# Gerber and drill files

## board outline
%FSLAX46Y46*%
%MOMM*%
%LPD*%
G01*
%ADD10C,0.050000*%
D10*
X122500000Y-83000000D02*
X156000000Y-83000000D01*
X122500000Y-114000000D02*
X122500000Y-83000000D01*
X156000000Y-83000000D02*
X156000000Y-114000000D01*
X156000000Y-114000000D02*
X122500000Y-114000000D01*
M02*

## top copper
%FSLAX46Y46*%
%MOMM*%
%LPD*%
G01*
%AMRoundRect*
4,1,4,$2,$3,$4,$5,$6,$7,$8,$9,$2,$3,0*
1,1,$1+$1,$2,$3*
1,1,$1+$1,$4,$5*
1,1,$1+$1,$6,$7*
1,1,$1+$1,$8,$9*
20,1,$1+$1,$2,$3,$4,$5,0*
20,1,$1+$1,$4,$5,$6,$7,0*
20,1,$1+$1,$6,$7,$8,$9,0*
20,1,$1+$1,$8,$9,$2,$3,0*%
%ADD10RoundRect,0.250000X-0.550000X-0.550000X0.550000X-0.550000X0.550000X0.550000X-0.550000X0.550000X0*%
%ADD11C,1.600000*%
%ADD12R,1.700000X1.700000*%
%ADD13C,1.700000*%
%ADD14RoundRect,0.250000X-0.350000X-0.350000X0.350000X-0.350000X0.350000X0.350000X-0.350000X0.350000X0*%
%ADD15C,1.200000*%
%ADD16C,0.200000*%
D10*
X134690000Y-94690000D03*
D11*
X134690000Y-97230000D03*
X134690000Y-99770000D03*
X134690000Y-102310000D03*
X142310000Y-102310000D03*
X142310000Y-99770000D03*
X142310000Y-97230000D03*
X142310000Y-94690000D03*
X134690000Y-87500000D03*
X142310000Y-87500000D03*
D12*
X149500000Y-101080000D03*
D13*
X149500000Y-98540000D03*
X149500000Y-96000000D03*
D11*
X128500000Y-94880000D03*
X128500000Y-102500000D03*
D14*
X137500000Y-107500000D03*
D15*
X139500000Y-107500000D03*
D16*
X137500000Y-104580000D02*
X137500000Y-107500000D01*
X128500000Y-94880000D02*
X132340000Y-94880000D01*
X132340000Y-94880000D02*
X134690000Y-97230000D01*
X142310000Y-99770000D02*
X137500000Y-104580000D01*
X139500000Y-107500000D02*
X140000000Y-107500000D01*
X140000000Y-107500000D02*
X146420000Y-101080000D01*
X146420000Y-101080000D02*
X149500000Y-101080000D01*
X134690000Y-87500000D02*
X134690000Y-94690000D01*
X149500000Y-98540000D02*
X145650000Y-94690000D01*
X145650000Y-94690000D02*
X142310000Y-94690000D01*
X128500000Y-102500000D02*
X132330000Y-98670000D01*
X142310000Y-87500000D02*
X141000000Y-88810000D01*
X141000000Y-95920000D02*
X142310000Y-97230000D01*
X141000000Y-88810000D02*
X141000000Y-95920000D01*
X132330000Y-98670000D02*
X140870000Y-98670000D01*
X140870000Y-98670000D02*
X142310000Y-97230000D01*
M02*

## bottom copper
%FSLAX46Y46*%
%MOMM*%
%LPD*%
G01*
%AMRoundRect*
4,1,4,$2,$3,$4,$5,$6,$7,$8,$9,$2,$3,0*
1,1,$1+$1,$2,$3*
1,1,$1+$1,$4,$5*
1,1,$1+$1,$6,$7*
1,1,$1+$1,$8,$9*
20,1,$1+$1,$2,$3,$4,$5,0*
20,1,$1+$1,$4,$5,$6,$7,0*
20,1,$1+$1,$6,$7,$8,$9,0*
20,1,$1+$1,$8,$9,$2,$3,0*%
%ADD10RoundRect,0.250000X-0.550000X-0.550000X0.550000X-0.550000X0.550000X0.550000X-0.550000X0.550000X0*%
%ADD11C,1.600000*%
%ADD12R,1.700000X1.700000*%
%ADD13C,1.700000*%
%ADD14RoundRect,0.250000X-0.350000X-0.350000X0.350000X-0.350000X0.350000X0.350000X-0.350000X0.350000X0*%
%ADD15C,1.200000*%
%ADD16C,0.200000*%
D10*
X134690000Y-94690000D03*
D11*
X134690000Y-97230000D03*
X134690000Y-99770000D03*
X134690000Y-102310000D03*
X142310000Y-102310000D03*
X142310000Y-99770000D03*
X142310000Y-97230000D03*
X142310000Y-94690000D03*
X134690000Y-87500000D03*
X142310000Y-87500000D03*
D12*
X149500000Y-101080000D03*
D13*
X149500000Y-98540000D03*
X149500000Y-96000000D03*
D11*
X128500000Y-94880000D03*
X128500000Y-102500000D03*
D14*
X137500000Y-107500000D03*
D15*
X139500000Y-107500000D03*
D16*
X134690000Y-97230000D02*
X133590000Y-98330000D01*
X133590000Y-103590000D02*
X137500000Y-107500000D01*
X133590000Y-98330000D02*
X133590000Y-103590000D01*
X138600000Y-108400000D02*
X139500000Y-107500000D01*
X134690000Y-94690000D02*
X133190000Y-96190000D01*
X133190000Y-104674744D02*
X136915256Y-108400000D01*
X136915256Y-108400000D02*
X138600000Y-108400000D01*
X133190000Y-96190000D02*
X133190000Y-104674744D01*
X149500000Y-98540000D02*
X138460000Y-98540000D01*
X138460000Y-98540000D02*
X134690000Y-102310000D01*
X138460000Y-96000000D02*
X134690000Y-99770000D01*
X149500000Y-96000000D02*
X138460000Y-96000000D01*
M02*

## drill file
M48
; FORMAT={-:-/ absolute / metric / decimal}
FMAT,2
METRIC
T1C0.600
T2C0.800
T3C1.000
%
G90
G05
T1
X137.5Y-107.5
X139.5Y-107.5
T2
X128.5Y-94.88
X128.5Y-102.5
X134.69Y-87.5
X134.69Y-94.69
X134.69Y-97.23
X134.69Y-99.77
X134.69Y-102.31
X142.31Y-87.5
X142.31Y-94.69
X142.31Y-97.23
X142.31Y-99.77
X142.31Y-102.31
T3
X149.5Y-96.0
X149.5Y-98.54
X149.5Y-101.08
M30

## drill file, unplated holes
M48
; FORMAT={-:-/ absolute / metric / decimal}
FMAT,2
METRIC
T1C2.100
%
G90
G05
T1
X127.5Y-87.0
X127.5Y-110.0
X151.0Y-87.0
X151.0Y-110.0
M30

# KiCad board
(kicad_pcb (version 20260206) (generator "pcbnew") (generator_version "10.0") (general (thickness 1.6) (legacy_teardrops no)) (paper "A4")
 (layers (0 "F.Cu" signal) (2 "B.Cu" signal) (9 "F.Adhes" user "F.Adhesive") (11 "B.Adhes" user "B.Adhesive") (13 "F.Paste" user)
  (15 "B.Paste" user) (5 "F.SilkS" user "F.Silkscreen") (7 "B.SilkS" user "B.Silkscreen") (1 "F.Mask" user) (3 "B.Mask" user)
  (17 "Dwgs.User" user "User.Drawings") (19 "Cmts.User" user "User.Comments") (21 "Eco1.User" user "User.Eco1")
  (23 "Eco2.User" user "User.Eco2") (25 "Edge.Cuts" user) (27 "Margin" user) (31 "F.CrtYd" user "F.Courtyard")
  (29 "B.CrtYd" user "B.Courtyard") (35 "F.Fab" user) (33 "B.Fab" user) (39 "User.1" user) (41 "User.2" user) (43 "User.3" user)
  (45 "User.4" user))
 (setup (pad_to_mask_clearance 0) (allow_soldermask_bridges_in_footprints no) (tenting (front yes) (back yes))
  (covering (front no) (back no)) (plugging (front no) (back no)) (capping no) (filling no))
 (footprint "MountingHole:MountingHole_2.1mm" (layer "F.Cu") (at 151 110)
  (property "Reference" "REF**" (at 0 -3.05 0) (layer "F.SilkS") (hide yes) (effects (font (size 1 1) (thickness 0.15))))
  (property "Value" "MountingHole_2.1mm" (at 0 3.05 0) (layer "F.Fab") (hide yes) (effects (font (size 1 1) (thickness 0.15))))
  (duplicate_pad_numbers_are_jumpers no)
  (pad "" np_thru_hole circle (at 0 0) (size 2.1 2.1) (drill 2.1) (layers "*.Cu" "*.Mask")))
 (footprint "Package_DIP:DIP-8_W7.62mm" (layer "F.Cu") (at 134.69 94.69)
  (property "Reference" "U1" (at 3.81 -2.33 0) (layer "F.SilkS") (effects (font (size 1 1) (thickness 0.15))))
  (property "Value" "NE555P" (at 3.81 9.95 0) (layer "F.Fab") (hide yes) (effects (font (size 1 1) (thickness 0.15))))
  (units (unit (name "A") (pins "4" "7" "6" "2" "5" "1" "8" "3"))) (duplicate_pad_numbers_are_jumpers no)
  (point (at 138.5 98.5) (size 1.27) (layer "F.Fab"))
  (pad "1" thru_hole roundrect (at 0 0) (size 1.6 1.6) (drill 0.8) (layers "*.Cu" "*.Mask") (remove_unused_layers no)
   (roundrect_rratio 0.15625) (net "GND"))
  (pad "2" thru_hole circle (at 0 2.54) (size 1.6 1.6) (drill 0.8) (layers "*.Cu" "*.Mask") (remove_unused_layers no) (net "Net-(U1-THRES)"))
  (pad "3" thru_hole circle (at 0 5.08) (size 1.6 1.6) (drill 0.8) (layers "*.Cu" "*.Mask") (remove_unused_layers no) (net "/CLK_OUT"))
  (pad "4" thru_hole circle (at 0 7.62) (size 1.6 1.6) (drill 0.8) (layers "*.Cu" "*.Mask") (remove_unused_layers no) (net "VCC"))
  (pad "5" thru_hole circle (at 7.62 7.62) (size 1.6 1.6) (drill 0.8) (layers "*.Cu" "*.Mask") (remove_unused_layers no)
   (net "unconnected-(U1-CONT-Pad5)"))
  (pad "6" thru_hole circle (at 7.62 5.08) (size 1.6 1.6) (drill 0.8) (layers "*.Cu" "*.Mask") (remove_unused_layers no)
   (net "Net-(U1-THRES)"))
  (pad "7" thru_hole circle (at 7.62 2.54) (size 1.6 1.6) (drill 0.8) (layers "*.Cu" "*.Mask") (remove_unused_layers no)
   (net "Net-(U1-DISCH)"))
  (pad "8" thru_hole circle (at 7.62 0) (size 1.6 1.6) (drill 0.8) (layers "*.Cu" "*.Mask") (remove_unused_layers no) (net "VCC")))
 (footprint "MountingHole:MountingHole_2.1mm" (layer "F.Cu") (at 151 87)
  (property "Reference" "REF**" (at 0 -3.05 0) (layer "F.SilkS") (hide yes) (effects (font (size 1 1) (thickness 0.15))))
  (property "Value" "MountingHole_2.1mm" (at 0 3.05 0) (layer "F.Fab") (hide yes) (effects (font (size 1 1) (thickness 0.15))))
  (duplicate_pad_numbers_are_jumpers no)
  (pad "" np_thru_hole circle (at 0 0) (size 2.1 2.1) (drill 2.1) (layers "*.Cu" "*.Mask")))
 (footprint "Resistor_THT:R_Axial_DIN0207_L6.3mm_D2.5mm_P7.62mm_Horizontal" (layer "F.Cu") (at 134.69 87.5)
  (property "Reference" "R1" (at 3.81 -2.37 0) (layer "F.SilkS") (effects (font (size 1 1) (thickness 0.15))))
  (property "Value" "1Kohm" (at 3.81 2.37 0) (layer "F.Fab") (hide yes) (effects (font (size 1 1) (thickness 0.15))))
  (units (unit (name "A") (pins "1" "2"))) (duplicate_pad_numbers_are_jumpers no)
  (pad "1" thru_hole circle (at 0 0) (size 1.6 1.6) (drill 0.8) (layers "*.Cu" "*.Mask") (remove_unused_layers no) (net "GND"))
  (pad "2" thru_hole circle (at 7.62 0) (size 1.6 1.6) (drill 0.8) (layers "*.Cu" "*.Mask") (remove_unused_layers no) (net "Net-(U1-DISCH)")))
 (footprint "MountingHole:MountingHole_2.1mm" (layer "F.Cu") (at 127.5 110)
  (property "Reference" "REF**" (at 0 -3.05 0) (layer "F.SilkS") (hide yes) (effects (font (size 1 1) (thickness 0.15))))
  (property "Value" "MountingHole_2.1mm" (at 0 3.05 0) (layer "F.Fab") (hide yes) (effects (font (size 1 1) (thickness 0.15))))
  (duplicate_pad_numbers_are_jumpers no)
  (pad "" np_thru_hole circle (at 0 0) (size 2.1 2.1) (drill 2.1) (layers "*.Cu" "*.Mask")))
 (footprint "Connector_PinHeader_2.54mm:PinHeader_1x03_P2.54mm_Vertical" (layer "F.Cu") (at 149.5 101.08 180)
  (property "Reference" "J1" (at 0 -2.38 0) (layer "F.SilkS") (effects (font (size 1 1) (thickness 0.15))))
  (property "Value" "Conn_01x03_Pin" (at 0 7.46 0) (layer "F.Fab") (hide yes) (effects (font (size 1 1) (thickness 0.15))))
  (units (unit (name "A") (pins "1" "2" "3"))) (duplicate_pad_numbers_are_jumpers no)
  (pad "1" thru_hole rect (at 0 0 180) (size 1.7 1.7) (drill 1) (layers "*.Cu" "*.Mask") (remove_unused_layers no) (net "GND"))
  (pad "2" thru_hole circle (at 0 2.54 180) (size 1.7 1.7) (drill 1) (layers "*.Cu" "*.Mask") (remove_unused_layers no) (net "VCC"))
  (pad "3" thru_hole circle (at 0 5.08 180) (size 1.7 1.7) (drill 1) (layers "*.Cu" "*.Mask") (remove_unused_layers no) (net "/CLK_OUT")))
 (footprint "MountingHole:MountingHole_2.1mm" (layer "F.Cu") (at 127.5 87)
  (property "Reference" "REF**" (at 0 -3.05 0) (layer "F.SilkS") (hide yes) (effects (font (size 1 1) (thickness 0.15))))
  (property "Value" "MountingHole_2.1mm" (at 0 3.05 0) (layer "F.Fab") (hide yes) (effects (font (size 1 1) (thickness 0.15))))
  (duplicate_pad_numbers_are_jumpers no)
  (pad "" np_thru_hole circle (at 0 0) (size 2.1 2.1) (drill 2.1) (layers "*.Cu" "*.Mask")))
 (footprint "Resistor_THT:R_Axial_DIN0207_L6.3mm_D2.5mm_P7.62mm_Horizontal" (layer "F.Cu") (at 128.5 94.88 -90)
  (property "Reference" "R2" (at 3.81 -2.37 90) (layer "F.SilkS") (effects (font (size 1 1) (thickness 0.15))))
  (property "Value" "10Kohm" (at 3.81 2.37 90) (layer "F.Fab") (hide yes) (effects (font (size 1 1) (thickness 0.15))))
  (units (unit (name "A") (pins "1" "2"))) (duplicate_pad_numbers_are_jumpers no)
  (pad "1" thru_hole circle (at 0 0 270) (size 1.6 1.6) (drill 0.8) (layers "*.Cu" "*.Mask") (remove_unused_layers no)
   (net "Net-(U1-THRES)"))
  (pad "2" thru_hole circle (at 7.62 0 270) (size 1.6 1.6) (drill 0.8) (layers "*.Cu" "*.Mask") (remove_unused_layers no)
   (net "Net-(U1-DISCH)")))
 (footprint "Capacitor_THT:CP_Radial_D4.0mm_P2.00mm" (layer "F.Cu") (at 137.5 107.5)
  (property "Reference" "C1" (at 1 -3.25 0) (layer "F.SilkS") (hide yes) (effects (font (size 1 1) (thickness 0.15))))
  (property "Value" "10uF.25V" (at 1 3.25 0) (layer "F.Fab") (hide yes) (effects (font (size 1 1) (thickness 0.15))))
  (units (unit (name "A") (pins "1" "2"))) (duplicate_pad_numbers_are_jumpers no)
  (pad "1" thru_hole roundrect (at 0 0) (size 1.2 1.2) (drill 0.6) (layers "*.Cu" "*.Mask") (remove_unused_layers no)
   (roundrect_rratio 0.208333) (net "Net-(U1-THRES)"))
  (pad "2" thru_hole circle (at 2 0) (size 1.2 1.2) (drill 0.6) (layers "*.Cu" "*.Mask") (remove_unused_layers no) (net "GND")))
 (gr_line (start 122.5 83) (end 156 83) (stroke (width 0.05) (type default)) (layer "Edge.Cuts"))
 (gr_line (start 122.5 114) (end 122.5 83) (stroke (width 0.05) (type default)) (layer "Edge.Cuts"))
 (gr_line (start 156 83) (end 156 114) (stroke (width 0.05) (type default)) (layer "Edge.Cuts"))
 (gr_line (start 156 114) (end 122.5 114) (stroke (width 0.05) (type default)) (layer "Edge.Cuts"))
 (segment (start 139.5 107.5) (end 140 107.5) (width 0.2) (layer "F.Cu") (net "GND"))
 (segment (start 140 107.5) (end 146.42 101.08) (width 0.2) (layer "F.Cu") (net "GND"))
 (segment (start 146.42 101.08) (end 149.5 101.08) (width 0.2) (layer "F.Cu") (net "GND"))
 (segment (start 134.69 87.5) (end 134.69 94.69) (width 0.2) (layer "F.Cu") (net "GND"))
 (segment (start 138.6 108.4) (end 139.5 107.5) (width 0.2) (layer "B.Cu") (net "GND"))
 (segment (start 134.69 94.69) (end 133.19 96.19) (width 0.2) (layer "B.Cu") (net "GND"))
 (segment (start 133.19 104.674744) (end 136.915256 108.4) (width 0.2) (layer "B.Cu") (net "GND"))
 (segment (start 136.915256 108.4) (end 138.6 108.4) (width 0.2) (layer "B.Cu") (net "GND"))
 (segment (start 133.19 96.19) (end 133.19 104.674744) (width 0.2) (layer "B.Cu") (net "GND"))
 (segment (start 137.5 104.58) (end 137.5 107.5) (width 0.2) (layer "F.Cu") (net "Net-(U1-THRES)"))
 (segment (start 128.5 94.88) (end 132.34 94.88) (width 0.2) (layer "F.Cu") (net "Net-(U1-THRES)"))
 (segment (start 132.34 94.88) (end 134.69 97.23) (width 0.2) (layer "F.Cu") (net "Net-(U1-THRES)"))
 (segment (start 142.31 99.77) (end 137.5 104.58) (width 0.2) (layer "F.Cu") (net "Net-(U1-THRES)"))
 (segment (start 134.69 97.23) (end 133.59 98.33) (width 0.2) (layer "B.Cu") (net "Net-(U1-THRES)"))
 (segment (start 133.59 103.59) (end 137.5 107.5) (width 0.2) (layer "B.Cu") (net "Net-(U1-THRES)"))
 (segment (start 133.59 98.33) (end 133.59 103.59) (width 0.2) (layer "B.Cu") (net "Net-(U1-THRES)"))
 (segment (start 138.46 96) (end 134.69 99.77) (width 0.2) (layer "B.Cu") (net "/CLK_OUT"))
 (segment (start 149.5 96) (end 138.46 96) (width 0.2) (layer "B.Cu") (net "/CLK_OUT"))
 (segment (start 149.5 98.54) (end 145.65 94.69) (width 0.2) (layer "F.Cu") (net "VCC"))
 (segment (start 145.65 94.69) (end 142.31 94.69) (width 0.2) (layer "F.Cu") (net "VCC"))
 (segment (start 149.5 98.54) (end 138.46 98.54) (width 0.2) (layer "B.Cu") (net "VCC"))
 (segment (start 138.46 98.54) (end 134.69 102.31) (width 0.2) (layer "B.Cu") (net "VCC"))
 (segment (start 128.5 102.5) (end 132.33 98.67) (width 0.2) (layer "F.Cu") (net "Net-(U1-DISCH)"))
 (segment (start 142.31 87.5) (end 141 88.81) (width 0.2) (layer "F.Cu") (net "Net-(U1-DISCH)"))
 (segment (start 141 95.92) (end 142.31 97.23) (width 0.2) (layer "F.Cu") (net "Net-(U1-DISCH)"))
 (segment (start 141 88.81) (end 141 95.92) (width 0.2) (layer "F.Cu") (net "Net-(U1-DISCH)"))
 (segment (start 132.33 98.67) (end 140.87 98.67) (width 0.2) (layer "F.Cu") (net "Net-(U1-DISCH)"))
 (segment (start 140.87 98.67) (end 142.31 97.23) (width 0.2) (layer "F.Cu") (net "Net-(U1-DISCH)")))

